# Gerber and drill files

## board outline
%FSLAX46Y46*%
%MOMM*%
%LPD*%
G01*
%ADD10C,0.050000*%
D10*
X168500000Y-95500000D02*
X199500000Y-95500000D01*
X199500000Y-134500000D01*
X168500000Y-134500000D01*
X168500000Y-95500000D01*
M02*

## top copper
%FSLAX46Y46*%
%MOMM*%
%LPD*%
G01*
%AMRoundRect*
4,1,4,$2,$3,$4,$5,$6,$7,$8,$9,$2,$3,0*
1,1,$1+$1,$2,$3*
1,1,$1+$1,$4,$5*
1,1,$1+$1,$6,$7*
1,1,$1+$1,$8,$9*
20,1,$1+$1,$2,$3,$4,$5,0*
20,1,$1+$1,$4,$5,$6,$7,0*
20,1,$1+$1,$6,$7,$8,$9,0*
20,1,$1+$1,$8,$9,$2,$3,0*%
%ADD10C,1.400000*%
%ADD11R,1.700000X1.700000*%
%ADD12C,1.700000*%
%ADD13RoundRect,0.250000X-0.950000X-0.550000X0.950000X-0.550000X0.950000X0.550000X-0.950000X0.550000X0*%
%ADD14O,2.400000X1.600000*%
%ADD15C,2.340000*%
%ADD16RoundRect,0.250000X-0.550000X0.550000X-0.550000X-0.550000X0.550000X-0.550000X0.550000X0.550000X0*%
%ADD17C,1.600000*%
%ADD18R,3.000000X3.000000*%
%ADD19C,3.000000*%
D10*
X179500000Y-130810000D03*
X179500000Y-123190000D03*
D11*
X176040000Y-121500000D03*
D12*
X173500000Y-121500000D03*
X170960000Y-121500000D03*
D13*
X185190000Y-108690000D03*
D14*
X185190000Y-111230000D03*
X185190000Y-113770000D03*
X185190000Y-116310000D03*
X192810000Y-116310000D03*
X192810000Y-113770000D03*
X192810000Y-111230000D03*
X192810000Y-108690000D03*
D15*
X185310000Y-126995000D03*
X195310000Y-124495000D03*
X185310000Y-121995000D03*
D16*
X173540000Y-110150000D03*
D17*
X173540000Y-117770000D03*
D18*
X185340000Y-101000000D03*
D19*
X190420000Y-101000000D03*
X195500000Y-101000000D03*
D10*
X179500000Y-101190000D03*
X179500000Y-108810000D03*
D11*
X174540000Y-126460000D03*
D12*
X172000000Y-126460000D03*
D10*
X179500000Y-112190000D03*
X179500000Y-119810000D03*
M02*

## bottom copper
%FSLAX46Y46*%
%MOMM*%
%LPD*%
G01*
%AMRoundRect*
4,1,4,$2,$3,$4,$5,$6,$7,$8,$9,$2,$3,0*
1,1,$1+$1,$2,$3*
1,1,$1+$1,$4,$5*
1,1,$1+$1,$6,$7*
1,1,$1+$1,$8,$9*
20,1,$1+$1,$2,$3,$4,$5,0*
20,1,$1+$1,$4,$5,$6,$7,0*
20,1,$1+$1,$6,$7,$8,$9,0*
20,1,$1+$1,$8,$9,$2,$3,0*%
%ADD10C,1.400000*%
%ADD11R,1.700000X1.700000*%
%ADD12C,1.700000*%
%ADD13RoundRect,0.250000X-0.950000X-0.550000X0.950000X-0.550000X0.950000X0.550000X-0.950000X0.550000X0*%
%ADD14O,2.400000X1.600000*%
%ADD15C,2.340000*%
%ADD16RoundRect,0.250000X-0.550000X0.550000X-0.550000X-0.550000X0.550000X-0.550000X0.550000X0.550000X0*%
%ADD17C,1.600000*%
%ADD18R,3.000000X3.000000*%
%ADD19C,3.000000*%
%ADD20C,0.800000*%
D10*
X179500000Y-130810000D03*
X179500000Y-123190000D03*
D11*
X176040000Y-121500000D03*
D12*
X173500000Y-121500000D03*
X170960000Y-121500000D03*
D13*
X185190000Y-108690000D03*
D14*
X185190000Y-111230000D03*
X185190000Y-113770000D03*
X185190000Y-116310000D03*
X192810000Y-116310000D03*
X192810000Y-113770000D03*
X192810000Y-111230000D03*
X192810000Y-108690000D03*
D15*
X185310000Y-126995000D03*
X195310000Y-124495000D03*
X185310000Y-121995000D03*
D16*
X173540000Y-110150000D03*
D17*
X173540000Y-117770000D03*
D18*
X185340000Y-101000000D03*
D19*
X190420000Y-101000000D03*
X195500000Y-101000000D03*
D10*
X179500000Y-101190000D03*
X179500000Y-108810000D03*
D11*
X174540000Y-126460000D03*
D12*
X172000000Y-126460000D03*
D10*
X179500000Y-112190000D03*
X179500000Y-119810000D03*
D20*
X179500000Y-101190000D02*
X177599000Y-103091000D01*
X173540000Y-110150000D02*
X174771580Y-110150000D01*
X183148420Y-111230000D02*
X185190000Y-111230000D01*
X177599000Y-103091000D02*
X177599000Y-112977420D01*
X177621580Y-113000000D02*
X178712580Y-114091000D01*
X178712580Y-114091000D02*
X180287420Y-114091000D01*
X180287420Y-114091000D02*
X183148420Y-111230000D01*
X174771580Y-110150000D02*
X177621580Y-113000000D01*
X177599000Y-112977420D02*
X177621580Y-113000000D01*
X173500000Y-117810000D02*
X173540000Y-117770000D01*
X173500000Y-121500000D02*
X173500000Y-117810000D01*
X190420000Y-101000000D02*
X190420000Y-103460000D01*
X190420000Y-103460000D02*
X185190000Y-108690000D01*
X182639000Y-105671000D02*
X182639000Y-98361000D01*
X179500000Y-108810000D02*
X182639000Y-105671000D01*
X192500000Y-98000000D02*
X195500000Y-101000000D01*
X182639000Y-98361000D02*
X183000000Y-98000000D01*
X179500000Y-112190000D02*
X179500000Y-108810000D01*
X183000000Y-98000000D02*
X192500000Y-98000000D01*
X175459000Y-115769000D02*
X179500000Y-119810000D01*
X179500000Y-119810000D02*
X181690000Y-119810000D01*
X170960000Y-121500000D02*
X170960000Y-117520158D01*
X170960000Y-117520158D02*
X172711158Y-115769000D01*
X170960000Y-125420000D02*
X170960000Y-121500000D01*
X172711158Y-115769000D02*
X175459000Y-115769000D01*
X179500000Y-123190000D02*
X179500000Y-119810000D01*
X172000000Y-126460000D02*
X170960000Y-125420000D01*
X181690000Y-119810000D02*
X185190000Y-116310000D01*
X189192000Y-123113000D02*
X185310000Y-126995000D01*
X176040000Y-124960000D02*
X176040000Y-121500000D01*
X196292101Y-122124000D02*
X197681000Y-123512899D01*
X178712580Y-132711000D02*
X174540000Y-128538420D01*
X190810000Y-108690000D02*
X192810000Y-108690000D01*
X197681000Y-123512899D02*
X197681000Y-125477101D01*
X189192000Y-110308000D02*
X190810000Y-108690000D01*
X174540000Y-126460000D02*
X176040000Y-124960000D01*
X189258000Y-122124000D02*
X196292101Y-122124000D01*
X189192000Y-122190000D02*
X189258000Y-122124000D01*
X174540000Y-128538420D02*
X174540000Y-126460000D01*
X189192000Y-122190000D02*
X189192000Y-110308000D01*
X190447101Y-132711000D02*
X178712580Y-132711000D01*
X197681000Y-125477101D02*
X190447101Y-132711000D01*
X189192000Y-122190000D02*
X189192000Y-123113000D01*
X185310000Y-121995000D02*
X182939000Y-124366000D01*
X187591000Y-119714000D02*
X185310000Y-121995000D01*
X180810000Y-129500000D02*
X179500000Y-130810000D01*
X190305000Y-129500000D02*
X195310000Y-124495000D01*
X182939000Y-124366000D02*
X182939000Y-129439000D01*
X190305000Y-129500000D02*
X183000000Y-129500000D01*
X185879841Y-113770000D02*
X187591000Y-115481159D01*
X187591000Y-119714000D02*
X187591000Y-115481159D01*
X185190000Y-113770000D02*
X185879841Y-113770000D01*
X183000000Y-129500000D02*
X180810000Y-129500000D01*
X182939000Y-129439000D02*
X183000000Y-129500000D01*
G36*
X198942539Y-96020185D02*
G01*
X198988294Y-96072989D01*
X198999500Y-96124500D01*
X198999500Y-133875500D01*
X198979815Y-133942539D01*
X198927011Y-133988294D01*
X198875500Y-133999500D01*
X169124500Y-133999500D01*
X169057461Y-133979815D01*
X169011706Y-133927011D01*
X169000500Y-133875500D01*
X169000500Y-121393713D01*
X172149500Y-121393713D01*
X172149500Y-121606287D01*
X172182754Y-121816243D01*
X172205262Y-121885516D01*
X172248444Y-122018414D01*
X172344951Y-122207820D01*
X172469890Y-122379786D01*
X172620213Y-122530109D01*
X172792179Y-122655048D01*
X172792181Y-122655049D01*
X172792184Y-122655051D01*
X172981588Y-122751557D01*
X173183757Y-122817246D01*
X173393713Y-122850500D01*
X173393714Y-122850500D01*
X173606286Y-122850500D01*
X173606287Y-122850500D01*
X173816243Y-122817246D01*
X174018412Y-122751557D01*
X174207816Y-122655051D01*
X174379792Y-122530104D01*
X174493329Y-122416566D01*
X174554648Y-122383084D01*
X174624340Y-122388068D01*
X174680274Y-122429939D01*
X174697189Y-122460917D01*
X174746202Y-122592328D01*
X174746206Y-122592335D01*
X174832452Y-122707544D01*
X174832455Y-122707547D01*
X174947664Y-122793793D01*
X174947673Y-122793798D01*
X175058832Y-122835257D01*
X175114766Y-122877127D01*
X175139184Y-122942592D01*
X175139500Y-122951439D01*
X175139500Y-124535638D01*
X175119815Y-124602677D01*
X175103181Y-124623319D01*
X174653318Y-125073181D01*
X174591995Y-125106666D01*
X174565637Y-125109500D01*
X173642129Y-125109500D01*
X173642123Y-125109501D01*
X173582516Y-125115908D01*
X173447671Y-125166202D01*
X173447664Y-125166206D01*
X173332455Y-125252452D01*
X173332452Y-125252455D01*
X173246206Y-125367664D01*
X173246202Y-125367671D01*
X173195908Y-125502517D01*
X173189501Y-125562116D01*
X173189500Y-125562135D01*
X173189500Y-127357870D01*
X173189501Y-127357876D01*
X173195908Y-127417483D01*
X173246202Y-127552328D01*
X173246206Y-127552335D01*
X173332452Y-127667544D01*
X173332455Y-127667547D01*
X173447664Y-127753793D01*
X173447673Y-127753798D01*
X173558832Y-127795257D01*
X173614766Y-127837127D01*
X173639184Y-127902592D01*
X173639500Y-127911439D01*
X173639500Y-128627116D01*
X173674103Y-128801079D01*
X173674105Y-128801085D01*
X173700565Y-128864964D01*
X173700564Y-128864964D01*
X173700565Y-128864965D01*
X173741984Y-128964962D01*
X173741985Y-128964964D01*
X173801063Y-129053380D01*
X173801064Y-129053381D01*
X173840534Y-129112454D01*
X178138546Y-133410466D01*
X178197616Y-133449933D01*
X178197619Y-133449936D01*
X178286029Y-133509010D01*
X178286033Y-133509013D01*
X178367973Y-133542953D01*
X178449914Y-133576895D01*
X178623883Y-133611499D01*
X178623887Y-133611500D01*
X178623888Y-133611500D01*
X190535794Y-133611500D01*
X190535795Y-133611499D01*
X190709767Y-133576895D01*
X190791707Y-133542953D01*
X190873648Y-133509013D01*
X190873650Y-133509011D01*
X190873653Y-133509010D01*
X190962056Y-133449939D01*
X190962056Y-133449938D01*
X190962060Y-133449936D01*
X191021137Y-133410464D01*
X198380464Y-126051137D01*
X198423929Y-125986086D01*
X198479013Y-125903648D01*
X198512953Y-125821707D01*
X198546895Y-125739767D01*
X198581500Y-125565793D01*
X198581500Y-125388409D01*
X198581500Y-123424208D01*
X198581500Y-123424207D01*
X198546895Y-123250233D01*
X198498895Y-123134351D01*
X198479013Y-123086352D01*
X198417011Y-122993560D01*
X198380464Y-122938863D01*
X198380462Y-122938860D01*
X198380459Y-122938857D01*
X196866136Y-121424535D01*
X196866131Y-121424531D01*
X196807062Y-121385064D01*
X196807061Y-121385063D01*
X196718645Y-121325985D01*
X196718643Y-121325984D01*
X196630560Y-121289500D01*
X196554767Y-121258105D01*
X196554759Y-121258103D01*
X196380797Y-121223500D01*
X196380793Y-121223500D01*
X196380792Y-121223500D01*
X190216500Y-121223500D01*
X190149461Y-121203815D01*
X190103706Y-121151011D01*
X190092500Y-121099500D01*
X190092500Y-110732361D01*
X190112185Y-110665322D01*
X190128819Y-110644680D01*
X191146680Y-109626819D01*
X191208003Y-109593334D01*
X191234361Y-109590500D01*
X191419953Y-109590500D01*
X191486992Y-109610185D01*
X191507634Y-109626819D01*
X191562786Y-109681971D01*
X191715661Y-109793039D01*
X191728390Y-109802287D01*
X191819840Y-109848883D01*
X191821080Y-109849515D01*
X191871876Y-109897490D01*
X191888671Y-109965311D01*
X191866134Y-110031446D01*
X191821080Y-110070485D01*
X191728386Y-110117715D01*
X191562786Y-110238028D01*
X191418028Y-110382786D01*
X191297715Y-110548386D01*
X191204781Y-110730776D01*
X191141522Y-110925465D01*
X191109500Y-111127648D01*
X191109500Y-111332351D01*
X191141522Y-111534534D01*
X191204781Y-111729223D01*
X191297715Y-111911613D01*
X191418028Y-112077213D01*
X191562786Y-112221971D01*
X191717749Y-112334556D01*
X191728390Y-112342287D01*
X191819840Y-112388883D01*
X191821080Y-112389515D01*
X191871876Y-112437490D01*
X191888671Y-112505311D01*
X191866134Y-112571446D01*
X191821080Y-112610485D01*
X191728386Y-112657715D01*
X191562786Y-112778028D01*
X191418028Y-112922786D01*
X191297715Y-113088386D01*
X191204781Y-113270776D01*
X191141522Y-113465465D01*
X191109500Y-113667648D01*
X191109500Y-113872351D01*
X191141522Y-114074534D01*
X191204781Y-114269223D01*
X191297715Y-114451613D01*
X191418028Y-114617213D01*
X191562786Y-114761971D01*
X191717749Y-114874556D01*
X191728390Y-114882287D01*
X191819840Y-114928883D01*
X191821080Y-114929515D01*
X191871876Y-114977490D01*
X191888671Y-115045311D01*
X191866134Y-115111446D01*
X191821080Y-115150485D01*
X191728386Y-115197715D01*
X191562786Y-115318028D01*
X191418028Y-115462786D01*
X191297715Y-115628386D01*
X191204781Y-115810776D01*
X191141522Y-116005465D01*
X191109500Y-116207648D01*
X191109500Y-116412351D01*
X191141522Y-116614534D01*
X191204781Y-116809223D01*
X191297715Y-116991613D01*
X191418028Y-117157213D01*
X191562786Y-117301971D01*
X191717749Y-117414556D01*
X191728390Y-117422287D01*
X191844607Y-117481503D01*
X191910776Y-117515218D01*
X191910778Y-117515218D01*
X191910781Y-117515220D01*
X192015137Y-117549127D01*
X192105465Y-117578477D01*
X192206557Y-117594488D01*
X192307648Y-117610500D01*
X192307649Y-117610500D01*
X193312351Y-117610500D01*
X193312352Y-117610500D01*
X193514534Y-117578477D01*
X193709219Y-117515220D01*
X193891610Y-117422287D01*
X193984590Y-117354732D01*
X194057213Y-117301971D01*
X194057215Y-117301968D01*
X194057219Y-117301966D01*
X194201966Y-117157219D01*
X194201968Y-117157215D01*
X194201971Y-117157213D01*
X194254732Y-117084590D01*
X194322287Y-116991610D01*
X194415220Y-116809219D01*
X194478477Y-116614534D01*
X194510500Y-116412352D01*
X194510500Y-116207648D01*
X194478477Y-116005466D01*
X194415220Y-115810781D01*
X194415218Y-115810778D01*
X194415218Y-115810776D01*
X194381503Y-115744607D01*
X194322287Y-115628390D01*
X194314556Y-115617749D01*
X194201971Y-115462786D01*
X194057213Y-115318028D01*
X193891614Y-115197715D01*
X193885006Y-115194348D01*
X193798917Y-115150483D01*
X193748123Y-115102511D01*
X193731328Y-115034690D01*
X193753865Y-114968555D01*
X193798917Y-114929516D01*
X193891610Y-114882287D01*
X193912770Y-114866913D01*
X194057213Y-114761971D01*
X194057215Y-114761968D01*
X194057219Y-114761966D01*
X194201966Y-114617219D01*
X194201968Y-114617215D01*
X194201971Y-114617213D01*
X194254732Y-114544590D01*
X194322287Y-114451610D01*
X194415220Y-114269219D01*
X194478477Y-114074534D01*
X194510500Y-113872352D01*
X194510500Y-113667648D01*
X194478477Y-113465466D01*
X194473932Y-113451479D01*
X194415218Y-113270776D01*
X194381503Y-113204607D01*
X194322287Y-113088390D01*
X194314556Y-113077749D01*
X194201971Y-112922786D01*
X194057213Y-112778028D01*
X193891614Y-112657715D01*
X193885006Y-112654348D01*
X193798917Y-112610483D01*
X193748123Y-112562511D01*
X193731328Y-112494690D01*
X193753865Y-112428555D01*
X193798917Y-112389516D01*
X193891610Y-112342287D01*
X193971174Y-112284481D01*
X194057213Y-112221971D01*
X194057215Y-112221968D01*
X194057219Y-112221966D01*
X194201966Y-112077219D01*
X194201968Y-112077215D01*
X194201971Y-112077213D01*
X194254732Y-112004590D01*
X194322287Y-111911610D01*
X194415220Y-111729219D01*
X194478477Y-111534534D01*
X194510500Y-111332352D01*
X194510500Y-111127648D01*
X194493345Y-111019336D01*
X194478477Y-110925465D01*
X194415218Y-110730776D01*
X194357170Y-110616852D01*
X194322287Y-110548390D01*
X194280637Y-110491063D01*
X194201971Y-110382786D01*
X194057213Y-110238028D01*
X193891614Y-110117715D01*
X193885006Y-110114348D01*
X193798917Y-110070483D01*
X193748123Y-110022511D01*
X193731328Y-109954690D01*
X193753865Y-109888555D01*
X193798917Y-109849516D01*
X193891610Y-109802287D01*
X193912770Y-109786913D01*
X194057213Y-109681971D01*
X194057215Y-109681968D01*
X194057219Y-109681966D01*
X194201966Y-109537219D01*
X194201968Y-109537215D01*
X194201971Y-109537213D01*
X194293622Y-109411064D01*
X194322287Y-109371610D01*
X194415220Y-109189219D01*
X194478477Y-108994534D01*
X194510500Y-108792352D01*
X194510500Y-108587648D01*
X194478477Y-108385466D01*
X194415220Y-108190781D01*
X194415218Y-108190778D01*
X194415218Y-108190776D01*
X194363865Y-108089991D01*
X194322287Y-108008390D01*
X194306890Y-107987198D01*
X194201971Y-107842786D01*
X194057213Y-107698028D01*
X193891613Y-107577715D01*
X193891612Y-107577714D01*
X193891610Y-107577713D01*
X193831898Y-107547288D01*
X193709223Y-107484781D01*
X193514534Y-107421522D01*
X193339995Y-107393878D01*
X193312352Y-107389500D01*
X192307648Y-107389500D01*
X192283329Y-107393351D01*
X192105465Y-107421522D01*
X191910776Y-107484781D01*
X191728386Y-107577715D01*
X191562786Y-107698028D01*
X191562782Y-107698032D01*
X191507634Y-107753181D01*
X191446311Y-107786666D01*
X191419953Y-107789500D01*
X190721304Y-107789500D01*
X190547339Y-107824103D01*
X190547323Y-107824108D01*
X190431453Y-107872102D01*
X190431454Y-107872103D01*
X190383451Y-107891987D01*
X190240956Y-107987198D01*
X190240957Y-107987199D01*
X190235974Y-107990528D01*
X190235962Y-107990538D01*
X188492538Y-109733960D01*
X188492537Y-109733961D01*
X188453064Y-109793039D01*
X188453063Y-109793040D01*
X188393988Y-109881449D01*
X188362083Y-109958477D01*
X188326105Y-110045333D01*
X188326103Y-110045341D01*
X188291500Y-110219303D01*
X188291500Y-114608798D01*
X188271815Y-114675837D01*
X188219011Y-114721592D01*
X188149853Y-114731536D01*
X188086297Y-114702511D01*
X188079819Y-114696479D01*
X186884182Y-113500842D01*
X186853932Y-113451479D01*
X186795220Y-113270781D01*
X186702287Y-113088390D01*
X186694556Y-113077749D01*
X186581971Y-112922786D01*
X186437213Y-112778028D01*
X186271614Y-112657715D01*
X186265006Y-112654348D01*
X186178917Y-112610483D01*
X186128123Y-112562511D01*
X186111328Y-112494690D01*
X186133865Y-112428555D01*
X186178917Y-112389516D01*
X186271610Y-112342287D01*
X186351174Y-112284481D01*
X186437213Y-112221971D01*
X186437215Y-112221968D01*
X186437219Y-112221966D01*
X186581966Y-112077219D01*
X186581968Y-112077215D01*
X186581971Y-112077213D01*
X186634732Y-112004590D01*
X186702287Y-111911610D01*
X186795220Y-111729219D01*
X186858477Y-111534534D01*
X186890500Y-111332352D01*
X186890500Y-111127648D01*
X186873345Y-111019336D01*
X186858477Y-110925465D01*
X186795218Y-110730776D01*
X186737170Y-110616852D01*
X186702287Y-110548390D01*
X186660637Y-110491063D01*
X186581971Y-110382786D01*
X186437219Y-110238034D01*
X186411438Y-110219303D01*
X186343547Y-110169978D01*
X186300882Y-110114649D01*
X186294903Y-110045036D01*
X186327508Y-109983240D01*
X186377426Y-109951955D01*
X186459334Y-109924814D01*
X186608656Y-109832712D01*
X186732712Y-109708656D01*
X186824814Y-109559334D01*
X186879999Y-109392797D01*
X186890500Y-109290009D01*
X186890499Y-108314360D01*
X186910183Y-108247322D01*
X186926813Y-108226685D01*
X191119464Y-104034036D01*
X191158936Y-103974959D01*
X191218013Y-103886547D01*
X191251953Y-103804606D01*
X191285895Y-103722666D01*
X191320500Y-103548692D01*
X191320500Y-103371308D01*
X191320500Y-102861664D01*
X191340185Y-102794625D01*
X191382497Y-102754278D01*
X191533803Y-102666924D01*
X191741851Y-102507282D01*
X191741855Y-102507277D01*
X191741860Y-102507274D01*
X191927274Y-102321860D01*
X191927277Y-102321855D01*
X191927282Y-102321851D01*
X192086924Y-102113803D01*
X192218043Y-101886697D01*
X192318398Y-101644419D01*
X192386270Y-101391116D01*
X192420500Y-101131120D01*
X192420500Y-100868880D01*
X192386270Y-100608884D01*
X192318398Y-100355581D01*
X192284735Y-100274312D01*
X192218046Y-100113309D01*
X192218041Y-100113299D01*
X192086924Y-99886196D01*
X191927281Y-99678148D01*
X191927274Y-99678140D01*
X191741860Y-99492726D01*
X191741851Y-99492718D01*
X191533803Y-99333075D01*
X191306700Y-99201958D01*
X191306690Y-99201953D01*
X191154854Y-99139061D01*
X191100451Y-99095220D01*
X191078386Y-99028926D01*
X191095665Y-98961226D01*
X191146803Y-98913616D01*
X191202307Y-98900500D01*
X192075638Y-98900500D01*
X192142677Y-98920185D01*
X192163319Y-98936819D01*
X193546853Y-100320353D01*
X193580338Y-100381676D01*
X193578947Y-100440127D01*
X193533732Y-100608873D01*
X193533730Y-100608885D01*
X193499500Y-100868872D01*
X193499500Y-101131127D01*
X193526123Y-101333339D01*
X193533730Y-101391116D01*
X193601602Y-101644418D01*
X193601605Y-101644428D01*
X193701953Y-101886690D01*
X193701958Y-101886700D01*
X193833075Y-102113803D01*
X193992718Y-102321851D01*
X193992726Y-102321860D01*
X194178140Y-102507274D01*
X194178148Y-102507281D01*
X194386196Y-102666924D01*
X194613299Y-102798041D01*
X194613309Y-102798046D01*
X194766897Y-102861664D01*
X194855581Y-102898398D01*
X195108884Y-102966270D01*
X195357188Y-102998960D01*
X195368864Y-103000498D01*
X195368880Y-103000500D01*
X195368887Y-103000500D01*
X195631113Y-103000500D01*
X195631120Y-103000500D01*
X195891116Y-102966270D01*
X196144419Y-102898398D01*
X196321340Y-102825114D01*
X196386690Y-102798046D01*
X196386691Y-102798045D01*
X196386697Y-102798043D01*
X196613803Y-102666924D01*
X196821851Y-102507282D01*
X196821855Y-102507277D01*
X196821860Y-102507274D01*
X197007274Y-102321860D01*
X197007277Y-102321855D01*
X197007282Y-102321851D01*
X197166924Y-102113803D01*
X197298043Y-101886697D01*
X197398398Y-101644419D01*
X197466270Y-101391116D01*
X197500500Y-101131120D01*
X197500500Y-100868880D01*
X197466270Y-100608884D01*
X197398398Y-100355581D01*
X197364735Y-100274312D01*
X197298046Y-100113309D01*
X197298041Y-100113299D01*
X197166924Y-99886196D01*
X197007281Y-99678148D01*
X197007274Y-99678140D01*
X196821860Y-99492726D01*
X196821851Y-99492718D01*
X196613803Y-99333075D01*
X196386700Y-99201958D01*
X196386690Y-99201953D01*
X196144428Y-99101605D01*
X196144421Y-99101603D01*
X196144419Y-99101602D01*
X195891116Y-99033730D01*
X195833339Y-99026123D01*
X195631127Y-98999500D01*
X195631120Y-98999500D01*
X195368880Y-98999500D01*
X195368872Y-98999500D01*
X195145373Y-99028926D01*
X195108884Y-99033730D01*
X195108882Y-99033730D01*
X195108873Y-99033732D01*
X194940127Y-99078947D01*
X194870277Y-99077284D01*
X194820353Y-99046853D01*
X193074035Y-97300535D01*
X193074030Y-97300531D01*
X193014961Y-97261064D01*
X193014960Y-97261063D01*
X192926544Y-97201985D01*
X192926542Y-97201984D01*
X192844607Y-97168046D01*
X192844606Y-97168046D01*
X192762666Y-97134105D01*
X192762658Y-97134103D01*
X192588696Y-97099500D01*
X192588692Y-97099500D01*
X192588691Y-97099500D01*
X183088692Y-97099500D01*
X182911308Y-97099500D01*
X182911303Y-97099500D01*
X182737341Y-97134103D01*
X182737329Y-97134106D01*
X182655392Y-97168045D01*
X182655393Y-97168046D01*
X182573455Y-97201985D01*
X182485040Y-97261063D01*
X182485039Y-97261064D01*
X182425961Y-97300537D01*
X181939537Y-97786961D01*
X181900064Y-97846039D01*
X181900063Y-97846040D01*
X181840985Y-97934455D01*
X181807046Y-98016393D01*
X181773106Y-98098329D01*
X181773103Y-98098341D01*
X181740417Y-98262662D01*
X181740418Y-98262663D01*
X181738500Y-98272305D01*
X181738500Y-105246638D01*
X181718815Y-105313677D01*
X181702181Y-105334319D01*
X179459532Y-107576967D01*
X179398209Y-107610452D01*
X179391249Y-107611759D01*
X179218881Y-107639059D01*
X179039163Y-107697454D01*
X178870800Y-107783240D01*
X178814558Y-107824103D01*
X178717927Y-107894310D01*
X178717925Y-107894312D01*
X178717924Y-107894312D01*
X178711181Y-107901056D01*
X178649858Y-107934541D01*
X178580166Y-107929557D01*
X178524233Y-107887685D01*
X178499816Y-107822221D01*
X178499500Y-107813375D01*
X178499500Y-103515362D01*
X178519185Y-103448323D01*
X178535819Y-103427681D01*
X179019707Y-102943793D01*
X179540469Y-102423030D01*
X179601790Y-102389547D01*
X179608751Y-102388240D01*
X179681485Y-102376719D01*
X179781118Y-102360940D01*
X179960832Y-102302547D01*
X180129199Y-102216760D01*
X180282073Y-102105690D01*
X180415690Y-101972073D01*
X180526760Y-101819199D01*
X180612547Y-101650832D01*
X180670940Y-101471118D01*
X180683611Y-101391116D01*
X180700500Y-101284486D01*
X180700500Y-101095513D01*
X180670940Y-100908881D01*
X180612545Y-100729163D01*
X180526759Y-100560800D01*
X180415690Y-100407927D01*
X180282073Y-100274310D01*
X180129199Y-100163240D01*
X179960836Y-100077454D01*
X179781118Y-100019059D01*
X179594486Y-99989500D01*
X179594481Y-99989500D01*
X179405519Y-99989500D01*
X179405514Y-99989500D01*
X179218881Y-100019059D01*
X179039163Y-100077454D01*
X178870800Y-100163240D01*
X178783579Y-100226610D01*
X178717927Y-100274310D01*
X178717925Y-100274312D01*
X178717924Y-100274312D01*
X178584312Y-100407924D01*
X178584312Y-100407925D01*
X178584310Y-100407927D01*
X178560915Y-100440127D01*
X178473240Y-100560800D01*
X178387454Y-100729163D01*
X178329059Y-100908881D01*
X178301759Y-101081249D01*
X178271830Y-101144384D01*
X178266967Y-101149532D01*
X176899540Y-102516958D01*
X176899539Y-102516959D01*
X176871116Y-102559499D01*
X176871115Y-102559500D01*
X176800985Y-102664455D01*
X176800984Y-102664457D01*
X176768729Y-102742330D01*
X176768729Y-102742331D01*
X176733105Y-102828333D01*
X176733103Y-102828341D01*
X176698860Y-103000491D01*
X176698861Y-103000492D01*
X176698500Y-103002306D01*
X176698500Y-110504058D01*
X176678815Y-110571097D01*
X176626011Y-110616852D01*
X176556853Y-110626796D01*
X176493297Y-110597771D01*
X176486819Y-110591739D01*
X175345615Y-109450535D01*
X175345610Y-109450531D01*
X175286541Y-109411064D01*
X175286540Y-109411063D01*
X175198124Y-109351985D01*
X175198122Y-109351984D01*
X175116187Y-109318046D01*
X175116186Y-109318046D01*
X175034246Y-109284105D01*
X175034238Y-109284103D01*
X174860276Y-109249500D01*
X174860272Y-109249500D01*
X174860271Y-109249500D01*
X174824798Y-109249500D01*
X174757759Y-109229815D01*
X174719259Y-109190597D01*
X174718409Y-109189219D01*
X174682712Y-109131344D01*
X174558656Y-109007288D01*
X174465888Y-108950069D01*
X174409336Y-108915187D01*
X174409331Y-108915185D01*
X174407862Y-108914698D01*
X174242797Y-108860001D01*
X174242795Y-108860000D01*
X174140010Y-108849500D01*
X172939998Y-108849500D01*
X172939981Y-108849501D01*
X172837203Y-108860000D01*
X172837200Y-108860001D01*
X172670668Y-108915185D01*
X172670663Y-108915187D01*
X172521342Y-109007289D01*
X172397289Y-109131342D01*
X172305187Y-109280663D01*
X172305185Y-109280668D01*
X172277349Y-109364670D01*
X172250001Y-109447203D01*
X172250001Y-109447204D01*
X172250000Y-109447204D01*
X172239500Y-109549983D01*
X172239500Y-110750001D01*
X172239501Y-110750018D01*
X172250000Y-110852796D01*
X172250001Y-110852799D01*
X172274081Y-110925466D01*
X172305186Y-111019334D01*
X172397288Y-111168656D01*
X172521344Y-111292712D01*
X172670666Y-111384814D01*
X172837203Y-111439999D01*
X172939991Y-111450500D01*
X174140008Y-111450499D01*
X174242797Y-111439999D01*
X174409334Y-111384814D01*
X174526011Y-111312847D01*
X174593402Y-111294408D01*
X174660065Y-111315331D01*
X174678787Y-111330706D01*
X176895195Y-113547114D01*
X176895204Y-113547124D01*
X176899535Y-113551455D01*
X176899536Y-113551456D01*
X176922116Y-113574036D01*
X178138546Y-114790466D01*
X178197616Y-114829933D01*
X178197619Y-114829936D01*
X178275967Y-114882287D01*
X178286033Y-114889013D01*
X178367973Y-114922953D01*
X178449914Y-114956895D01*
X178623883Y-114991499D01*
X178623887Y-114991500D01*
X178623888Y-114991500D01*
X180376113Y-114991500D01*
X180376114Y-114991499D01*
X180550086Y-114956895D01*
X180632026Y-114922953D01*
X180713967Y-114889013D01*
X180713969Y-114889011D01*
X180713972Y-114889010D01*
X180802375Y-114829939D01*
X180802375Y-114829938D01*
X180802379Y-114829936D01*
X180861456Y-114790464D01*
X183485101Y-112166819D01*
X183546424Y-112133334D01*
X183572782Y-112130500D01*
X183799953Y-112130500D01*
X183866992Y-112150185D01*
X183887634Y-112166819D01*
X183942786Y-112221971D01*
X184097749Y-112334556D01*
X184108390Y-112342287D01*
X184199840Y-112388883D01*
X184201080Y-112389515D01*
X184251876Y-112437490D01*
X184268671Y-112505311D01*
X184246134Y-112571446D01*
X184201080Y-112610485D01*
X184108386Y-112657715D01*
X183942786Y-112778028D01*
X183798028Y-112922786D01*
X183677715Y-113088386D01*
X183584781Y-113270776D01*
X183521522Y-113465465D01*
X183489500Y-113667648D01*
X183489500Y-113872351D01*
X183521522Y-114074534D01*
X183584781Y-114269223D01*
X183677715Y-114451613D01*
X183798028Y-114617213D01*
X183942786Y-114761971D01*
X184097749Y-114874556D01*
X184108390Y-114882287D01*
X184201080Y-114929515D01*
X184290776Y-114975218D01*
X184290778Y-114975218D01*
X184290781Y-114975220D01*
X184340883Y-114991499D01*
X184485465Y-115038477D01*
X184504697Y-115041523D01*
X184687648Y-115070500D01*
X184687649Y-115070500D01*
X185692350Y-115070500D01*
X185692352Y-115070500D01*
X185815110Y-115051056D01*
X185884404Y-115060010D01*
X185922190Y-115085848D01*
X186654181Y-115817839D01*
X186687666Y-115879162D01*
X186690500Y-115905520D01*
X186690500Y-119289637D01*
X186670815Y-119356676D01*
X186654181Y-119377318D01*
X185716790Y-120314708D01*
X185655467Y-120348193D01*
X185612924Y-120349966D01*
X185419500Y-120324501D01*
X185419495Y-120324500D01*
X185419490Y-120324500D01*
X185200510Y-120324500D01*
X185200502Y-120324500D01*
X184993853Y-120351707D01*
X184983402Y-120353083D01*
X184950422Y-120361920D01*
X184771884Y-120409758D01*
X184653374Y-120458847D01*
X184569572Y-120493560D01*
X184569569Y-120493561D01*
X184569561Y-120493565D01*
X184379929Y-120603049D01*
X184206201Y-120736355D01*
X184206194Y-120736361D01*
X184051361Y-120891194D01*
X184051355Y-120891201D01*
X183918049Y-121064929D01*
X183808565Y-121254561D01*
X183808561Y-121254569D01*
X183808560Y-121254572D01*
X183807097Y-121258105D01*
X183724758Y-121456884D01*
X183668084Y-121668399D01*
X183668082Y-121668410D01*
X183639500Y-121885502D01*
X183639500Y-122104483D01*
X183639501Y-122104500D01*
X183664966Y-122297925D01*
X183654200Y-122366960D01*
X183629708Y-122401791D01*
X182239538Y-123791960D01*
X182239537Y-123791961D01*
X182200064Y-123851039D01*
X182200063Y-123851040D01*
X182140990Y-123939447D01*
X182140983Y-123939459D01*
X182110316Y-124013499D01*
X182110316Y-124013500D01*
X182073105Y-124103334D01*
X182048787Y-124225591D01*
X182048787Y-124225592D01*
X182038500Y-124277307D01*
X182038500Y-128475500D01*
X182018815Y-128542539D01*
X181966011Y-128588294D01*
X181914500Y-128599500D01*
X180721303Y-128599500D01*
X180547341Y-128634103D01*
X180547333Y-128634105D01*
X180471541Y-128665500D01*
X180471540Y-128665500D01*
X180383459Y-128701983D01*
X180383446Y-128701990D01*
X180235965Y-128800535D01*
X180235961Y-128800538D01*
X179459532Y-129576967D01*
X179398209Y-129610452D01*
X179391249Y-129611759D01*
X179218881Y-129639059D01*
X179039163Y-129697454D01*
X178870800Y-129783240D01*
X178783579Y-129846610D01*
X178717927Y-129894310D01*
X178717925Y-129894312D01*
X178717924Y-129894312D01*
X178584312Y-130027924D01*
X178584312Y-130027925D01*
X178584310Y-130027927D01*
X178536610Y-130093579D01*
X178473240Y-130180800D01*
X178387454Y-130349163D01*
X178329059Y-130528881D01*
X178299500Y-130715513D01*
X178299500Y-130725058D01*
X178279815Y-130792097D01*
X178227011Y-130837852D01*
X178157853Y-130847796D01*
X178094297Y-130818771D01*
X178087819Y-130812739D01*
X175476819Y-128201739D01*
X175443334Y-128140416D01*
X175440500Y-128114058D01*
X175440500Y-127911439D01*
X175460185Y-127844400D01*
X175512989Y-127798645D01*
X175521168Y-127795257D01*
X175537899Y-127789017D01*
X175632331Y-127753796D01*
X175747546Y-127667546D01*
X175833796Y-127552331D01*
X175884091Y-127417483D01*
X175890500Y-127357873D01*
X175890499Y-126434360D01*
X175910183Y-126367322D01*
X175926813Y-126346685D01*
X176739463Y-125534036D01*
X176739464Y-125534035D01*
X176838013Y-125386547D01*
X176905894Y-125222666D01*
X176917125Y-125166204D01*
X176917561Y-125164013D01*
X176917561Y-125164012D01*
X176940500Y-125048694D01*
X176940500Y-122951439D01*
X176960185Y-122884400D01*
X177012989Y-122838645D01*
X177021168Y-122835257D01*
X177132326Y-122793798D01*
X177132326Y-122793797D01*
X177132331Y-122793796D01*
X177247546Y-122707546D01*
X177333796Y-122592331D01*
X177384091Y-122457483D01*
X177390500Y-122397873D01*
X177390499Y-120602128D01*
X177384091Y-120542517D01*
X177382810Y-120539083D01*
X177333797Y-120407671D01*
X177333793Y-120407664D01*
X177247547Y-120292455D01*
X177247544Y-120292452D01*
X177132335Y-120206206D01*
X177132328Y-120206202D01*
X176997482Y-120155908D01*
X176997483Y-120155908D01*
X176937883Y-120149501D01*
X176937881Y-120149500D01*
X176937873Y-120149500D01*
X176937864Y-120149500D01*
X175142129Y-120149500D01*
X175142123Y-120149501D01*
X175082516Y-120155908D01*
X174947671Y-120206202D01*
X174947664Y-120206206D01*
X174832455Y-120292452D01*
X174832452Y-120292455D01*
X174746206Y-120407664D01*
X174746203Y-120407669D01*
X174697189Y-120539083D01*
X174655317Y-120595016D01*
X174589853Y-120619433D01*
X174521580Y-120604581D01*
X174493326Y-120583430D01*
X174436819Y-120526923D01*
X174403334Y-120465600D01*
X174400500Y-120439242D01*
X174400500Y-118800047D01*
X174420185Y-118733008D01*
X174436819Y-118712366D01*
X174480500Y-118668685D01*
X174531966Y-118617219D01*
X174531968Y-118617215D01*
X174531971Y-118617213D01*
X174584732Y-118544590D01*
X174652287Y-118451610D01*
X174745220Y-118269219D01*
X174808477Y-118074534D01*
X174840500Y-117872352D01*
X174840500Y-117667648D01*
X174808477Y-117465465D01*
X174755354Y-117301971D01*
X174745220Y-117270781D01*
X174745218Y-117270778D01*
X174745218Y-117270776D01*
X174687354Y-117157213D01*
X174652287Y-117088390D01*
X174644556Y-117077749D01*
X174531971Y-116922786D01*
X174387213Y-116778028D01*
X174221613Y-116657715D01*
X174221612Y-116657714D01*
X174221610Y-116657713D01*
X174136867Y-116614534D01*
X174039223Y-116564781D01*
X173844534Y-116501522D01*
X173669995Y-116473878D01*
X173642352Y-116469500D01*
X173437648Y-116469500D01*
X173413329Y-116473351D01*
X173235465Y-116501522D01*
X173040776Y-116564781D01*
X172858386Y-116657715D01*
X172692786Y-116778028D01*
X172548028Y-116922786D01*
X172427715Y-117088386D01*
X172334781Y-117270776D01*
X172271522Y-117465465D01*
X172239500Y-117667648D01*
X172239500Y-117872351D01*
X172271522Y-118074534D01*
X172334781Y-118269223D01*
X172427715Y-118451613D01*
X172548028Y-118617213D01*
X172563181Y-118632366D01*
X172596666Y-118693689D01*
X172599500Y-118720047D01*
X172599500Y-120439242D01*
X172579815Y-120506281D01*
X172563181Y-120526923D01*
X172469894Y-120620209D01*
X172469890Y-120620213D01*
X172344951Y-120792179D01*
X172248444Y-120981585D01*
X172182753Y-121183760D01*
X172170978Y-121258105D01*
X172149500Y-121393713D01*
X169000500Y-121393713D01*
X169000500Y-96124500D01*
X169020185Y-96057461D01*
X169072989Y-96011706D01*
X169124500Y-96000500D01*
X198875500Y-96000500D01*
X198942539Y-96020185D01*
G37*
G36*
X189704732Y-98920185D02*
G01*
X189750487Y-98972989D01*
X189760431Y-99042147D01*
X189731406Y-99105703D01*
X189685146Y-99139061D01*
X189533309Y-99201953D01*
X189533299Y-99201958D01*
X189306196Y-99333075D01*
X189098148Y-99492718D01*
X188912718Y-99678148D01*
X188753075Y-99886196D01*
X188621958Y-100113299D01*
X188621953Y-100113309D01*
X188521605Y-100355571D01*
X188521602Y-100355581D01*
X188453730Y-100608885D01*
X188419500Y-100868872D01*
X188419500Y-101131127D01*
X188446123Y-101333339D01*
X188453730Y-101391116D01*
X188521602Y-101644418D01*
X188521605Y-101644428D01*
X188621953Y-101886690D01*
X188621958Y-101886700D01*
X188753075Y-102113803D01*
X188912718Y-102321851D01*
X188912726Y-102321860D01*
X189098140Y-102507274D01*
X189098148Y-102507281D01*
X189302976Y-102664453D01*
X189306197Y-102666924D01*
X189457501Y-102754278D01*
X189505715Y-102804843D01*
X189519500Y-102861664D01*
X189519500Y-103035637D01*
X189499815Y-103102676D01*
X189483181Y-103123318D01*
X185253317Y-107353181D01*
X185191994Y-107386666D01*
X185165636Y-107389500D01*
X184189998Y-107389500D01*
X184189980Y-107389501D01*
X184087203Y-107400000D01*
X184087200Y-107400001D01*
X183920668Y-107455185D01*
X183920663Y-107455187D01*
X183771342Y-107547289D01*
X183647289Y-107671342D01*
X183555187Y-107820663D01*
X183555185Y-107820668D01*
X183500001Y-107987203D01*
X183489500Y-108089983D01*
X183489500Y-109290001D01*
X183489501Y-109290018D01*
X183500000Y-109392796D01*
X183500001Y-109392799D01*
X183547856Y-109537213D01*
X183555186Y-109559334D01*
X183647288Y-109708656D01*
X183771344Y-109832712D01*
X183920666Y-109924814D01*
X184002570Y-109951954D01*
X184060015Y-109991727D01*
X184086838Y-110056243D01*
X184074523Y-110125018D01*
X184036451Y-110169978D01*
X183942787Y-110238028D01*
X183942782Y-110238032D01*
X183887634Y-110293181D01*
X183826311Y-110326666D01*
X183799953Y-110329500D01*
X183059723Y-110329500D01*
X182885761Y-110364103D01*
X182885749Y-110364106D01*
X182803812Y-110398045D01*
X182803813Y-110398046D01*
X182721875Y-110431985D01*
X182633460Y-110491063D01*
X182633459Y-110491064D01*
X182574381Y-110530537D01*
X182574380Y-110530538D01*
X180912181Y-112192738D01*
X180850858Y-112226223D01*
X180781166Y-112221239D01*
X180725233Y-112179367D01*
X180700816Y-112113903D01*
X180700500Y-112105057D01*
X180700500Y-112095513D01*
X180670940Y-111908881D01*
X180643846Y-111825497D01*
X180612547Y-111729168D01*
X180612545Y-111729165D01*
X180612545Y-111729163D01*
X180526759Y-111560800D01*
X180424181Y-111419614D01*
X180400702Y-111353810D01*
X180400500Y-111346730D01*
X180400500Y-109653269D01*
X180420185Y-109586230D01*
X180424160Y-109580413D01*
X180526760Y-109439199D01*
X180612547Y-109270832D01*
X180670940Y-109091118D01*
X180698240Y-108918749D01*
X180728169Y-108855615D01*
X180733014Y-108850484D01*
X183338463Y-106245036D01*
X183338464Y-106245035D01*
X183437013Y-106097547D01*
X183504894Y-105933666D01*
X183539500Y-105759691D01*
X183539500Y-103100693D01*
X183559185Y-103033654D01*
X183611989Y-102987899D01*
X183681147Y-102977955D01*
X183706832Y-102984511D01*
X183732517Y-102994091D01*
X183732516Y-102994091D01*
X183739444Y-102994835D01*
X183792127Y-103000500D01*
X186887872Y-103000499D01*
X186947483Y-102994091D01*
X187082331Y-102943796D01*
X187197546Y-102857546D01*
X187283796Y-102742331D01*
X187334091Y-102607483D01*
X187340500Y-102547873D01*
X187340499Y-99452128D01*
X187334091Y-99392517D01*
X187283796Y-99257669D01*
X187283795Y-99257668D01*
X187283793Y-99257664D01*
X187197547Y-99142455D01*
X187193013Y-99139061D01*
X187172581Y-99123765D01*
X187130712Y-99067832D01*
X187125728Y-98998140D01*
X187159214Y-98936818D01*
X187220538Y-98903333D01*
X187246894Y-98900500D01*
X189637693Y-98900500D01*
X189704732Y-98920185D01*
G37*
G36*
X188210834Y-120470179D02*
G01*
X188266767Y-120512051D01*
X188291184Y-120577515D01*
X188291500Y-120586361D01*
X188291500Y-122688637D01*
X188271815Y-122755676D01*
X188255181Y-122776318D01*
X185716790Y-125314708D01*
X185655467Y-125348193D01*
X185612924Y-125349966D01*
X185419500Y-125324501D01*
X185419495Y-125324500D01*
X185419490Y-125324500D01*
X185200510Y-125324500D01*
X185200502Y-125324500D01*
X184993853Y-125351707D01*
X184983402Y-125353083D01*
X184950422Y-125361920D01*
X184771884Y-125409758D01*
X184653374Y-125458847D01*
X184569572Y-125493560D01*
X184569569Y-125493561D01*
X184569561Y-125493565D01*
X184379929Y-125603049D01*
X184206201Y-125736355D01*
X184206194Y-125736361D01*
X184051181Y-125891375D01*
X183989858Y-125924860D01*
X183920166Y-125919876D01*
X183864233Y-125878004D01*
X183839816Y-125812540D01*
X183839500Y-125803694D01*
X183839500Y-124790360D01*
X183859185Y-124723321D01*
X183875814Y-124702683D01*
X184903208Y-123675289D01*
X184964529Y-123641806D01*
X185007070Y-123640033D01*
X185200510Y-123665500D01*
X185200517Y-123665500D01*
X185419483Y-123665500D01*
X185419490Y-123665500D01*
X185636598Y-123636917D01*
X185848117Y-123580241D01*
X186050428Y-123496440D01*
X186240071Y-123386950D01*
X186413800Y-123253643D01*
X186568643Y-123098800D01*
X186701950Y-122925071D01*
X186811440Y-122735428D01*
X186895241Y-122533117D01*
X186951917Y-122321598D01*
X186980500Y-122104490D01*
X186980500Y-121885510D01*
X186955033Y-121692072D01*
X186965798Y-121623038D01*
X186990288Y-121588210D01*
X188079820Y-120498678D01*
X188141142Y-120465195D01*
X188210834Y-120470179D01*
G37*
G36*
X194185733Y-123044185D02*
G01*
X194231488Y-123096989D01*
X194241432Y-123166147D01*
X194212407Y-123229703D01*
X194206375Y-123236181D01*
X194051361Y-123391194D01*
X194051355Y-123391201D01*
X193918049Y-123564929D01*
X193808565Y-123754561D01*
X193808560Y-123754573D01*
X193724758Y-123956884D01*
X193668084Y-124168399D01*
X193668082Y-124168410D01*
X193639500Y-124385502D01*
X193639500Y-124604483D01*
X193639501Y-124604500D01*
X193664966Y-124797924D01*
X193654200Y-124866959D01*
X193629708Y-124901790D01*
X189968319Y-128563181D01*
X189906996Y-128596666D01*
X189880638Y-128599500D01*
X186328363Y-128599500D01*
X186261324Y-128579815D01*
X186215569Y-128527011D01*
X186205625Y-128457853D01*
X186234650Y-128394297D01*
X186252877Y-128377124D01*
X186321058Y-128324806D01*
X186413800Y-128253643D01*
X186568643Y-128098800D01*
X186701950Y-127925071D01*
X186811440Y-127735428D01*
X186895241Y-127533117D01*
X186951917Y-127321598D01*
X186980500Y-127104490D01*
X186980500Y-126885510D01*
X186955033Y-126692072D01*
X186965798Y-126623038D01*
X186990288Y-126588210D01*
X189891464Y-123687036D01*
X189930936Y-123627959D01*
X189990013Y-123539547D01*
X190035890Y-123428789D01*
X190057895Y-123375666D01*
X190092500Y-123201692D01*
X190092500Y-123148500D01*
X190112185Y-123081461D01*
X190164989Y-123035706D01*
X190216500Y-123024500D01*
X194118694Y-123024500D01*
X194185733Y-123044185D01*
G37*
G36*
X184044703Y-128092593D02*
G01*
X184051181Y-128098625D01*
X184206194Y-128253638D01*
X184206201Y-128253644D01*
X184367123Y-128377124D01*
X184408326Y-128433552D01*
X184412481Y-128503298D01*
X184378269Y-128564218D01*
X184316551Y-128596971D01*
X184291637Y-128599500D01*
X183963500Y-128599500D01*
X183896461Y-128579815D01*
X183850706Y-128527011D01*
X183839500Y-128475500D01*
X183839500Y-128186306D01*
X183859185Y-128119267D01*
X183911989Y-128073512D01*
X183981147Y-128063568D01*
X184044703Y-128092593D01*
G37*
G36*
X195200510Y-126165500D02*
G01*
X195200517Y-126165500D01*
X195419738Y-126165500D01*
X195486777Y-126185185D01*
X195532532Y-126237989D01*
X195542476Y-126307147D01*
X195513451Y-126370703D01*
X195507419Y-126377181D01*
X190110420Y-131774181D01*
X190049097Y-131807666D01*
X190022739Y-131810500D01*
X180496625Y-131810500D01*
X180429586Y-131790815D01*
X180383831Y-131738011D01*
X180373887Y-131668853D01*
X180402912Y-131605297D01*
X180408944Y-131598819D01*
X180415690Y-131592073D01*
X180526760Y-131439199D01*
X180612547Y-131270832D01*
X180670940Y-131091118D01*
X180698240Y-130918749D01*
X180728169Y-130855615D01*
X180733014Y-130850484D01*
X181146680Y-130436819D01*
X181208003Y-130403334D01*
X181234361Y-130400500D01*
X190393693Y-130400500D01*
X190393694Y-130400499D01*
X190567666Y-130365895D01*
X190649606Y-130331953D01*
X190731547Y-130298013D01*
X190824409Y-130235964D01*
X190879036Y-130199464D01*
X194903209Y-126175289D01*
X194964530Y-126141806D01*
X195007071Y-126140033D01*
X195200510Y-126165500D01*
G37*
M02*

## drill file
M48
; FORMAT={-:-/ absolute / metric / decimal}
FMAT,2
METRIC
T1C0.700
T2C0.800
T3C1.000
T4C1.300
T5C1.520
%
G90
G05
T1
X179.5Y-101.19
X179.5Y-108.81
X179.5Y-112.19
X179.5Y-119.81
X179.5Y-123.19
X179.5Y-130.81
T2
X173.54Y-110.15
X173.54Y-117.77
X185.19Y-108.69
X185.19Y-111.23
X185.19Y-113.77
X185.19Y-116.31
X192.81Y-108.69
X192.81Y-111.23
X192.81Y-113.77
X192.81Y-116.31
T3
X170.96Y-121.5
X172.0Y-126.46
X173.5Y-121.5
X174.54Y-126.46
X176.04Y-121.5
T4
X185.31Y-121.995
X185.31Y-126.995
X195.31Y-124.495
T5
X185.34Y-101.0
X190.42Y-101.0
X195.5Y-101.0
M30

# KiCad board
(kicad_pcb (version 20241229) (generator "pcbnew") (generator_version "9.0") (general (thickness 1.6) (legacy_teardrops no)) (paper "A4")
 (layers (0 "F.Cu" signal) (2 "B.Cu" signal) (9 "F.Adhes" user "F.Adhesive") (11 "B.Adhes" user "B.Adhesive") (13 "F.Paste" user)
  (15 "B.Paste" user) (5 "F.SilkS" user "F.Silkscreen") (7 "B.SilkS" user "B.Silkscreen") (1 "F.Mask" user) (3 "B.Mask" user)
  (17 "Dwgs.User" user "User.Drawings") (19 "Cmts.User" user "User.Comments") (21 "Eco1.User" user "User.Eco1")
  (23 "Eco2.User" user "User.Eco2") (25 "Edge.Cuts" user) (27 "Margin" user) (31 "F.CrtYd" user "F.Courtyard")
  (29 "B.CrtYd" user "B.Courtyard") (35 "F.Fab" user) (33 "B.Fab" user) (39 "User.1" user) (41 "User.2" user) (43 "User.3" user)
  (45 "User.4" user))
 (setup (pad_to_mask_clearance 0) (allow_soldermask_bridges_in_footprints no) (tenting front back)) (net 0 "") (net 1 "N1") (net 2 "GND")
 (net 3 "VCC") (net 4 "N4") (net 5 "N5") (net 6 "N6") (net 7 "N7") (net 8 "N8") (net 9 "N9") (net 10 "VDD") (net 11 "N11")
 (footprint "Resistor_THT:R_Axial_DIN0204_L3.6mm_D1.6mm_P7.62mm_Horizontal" (layer "F.Cu") (at 179.5 130.81 90)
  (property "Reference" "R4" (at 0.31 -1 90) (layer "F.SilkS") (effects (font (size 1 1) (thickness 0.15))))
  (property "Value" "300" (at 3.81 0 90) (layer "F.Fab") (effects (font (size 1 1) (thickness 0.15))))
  (pad "1" thru_hole circle (at 0 0 90) (size 1.4 1.4) (drill 0.7) (layers "*.Cu" "*.Mask") (remove_unused_layers no) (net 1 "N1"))
  (pad "2" thru_hole circle (at 7.62 0 90) (size 1.4 1.4) (drill 0.7) (layers "*.Cu" "*.Mask") (remove_unused_layers no) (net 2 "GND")))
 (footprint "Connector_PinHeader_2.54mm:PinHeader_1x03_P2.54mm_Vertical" (layer "F.Cu") (at 176.04 121.5 -90)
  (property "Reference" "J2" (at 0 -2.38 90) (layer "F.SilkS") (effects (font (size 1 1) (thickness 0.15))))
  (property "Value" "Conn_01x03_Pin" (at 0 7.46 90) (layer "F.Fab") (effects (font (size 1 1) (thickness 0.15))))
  (pad "1" thru_hole rect (at 0 0 270) (size 1.7 1.7) (drill 1) (layers "*.Cu" "*.Mask") (remove_unused_layers no) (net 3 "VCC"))
  (pad "2" thru_hole circle (at 0 2.54 270) (size 1.7 1.7) (drill 1) (layers "*.Cu" "*.Mask") (remove_unused_layers no) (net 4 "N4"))
  (pad "3" thru_hole circle (at 0 5.08 270) (size 1.7 1.7) (drill 1) (layers "*.Cu" "*.Mask") (remove_unused_layers no) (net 2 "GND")))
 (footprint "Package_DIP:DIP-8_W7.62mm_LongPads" (layer "F.Cu") (at 185.19 108.69)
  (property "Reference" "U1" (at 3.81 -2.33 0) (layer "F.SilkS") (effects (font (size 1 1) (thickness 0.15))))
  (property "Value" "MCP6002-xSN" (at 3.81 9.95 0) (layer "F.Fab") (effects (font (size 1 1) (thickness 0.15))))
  (pad "1" thru_hole roundrect (at 0 0) (size 2.4 1.6) (drill 0.8) (layers "*.Cu" "*.Mask") (remove_unused_layers no)
   (roundrect_rratio 0.15625) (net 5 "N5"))
  (pad "2" thru_hole oval (at 0 2.54) (size 2.4 1.6) (drill 0.8) (layers "*.Cu" "*.Mask") (remove_unused_layers no) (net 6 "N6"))
  (pad "3" thru_hole oval (at 0 5.08) (size 2.4 1.6) (drill 0.8) (layers "*.Cu" "*.Mask") (remove_unused_layers no) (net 1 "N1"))
  (pad "4" thru_hole oval (at 0 7.62) (size 2.4 1.6) (drill 0.8) (layers "*.Cu" "*.Mask") (remove_unused_layers no) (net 2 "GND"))
  (pad "5" thru_hole oval (at 7.62 7.62) (size 2.4 1.6) (drill 0.8) (layers "*.Cu" "*.Mask") (remove_unused_layers no) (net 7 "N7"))
  (pad "6" thru_hole oval (at 7.62 5.08) (size 2.4 1.6) (drill 0.8) (layers "*.Cu" "*.Mask") (remove_unused_layers no) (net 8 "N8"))
  (pad "7" thru_hole oval (at 7.62 2.54) (size 2.4 1.6) (drill 0.8) (layers "*.Cu" "*.Mask") (remove_unused_layers no) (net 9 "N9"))
  (pad "8" thru_hole oval (at 7.62 0) (size 2.4 1.6) (drill 0.8) (layers "*.Cu" "*.Mask") (remove_unused_layers no) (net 3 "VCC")))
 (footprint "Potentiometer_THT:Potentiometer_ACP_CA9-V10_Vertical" (layer "F.Cu") (at 185.31 126.995)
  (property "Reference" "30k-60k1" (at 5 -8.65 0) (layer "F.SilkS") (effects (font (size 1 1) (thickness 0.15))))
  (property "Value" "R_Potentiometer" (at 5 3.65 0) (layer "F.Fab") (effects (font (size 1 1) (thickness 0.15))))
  (pad "1" thru_hole circle (at 0 0) (size 2.34 2.34) (drill 1.3) (layers "*.Cu" "*.Mask") (remove_unused_layers no) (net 3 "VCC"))
  (pad "2" thru_hole circle (at 10 -2.5) (size 2.34 2.34) (drill 1.3) (layers "*.Cu" "*.Mask") (remove_unused_layers no) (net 1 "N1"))
  (pad "3" thru_hole circle (at 0 -5) (size 2.34 2.34) (drill 1.3) (layers "*.Cu" "*.Mask") (remove_unused_layers no) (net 1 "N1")))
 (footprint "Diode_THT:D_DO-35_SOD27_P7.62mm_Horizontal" (layer "F.Cu") (at 173.54 110.15 -90)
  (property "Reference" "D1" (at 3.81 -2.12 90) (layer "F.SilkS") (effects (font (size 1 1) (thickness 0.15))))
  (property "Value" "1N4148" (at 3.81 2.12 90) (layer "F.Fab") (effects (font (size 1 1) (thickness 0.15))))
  (pad "1" thru_hole roundrect (at 0 0 270) (size 1.6 1.6) (drill 0.8) (layers "*.Cu" "*.Mask") (remove_unused_layers no)
   (roundrect_rratio 0.15625) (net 6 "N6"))
  (pad "2" thru_hole circle (at 7.62 0 270) (size 1.6 1.6) (drill 0.8) (layers "*.Cu" "*.Mask") (remove_unused_layers no) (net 4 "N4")))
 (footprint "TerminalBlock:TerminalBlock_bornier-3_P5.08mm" (layer "F.Cu") (at 185.34 101)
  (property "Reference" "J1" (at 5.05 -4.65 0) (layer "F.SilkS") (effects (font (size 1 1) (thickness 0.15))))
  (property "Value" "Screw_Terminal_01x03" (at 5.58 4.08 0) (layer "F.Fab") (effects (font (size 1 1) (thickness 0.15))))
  (pad "1" thru_hole rect (at 0 0) (size 3 3) (drill 1.52) (layers "*.Cu" "*.Mask") (remove_unused_layers no) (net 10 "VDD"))
  (pad "2" thru_hole circle (at 5.08 0) (size 3 3) (drill 1.52) (layers "*.Cu" "*.Mask") (remove_unused_layers no) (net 5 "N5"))
  (pad "3" thru_hole circle (at 10.16 0) (size 3 3) (drill 1.52) (layers "*.Cu" "*.Mask") (remove_unused_layers no) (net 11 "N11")))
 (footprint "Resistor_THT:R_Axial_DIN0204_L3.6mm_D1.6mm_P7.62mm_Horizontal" (layer "F.Cu") (at 179.5 101.19 -90)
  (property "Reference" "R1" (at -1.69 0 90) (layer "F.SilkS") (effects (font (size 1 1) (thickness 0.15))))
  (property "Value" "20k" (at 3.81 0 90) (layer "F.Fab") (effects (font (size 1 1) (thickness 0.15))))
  (pad "1" thru_hole circle (at 0 0 270) (size 1.4 1.4) (drill 0.7) (layers "*.Cu" "*.Mask") (remove_unused_layers no) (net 6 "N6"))
  (pad "2" thru_hole circle (at 7.62 0 270) (size 1.4 1.4) (drill 0.7) (layers "*.Cu" "*.Mask") (remove_unused_layers no) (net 11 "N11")))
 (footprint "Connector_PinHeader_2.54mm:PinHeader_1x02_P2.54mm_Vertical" (layer "F.Cu") (at 174.54 126.46 -90)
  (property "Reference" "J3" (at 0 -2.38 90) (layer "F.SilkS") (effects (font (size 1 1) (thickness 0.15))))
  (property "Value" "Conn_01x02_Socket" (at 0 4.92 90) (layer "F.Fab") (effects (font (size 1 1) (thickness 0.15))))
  (pad "1" thru_hole rect (at 0 0 270) (size 1.7 1.7) (drill 1) (layers "*.Cu" "*.Mask") (remove_unused_layers no) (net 3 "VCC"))
  (pad "2" thru_hole circle (at 0 2.54 270) (size 1.7 1.7) (drill 1) (layers "*.Cu" "*.Mask") (remove_unused_layers no) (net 2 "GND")))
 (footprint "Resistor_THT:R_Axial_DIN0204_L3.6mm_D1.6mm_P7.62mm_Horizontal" (layer "F.Cu") (at 179.5 112.19 -90)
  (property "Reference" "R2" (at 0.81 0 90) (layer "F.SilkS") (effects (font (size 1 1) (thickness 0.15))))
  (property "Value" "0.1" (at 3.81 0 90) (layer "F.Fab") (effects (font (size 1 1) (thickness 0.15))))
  (pad "1" thru_hole circle (at 0 0 270) (size 1.4 1.4) (drill 0.7) (layers "*.Cu" "*.Mask") (remove_unused_layers no) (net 11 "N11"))
  (pad "2" thru_hole circle (at 7.62 0 270) (size 1.4 1.4) (drill 0.7) (layers "*.Cu" "*.Mask") (remove_unused_layers no) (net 2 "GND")))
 (gr_rect (start 168.5 95.5) (end 199.5 134.5) (stroke (width 0.05) (type default)) (fill no) (layer "Edge.Cuts"))
 (segment (start 179.5 101.19) (end 177.599 103.091) (width 0.8) (layer "B.Cu") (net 6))
 (segment (start 173.54 110.15) (end 174.77158 110.15) (width 0.8) (layer "B.Cu") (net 6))
 (segment (start 183.14842 111.23) (end 185.19 111.23) (width 0.8) (layer "B.Cu") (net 6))
 (segment (start 177.599 103.091) (end 177.599 112.97742) (width 0.8) (layer "B.Cu") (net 6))
 (segment (start 177.62158 113) (end 178.71258 114.091) (width 0.8) (layer "B.Cu") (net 6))
 (segment (start 178.71258 114.091) (end 180.28742 114.091) (width 0.8) (layer "B.Cu") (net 6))
 (segment (start 180.28742 114.091) (end 183.14842 111.23) (width 0.8) (layer "B.Cu") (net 6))
 (segment (start 174.77158 110.15) (end 177.62158 113) (width 0.8) (layer "B.Cu") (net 6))
 (segment (start 177.599 112.97742) (end 177.62158 113) (width 0.8) (layer "B.Cu") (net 6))
 (segment (start 173.5 117.81) (end 173.54 117.77) (width 0.8) (layer "B.Cu") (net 4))
 (segment (start 173.5 121.5) (end 173.5 117.81) (width 0.8) (layer "B.Cu") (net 4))
 (segment (start 190.42 101) (end 190.42 103.46) (width 0.8) (layer "B.Cu") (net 5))
 (segment (start 190.42 103.46) (end 185.19 108.69) (width 0.8) (layer "B.Cu") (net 5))
 (segment (start 182.639 105.671) (end 182.639 98.361) (width 0.8) (layer "B.Cu") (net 11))
 (segment (start 179.5 108.81) (end 182.639 105.671) (width 0.8) (layer "B.Cu") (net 11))
 (segment (start 192.5 98) (end 195.5 101) (width 0.8) (layer "B.Cu") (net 11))
 (segment (start 182.639 98.361) (end 183 98) (width 0.8) (layer "B.Cu") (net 11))
 (segment (start 179.5 112.19) (end 179.5 108.81) (width 0.8) (layer "B.Cu") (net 11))
 (segment (start 183 98) (end 192.5 98) (width 0.8) (layer "B.Cu") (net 11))
 (segment (start 175.459 115.769) (end 179.5 119.81) (width 0.8) (layer "B.Cu") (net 2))
 (segment (start 179.5 119.81) (end 181.69 119.81) (width 0.8) (layer "B.Cu") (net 2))
 (segment (start 170.96 121.5) (end 170.96 117.520158) (width 0.8) (layer "B.Cu") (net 2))
 (segment (start 170.96 117.520158) (end 172.711158 115.769) (width 0.8) (layer "B.Cu") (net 2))
 (segment (start 170.96 125.42) (end 170.96 121.5) (width 0.8) (layer "B.Cu") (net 2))
 (segment (start 172.711158 115.769) (end 175.459 115.769) (width 0.8) (layer "B.Cu") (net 2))
 (segment (start 179.5 123.19) (end 179.5 119.81) (width 0.8) (layer "B.Cu") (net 2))
 (segment (start 172 126.46) (end 170.96 125.42) (width 0.8) (layer "B.Cu") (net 2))
 (segment (start 181.69 119.81) (end 185.19 116.31) (width 0.8) (layer "B.Cu") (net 2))
 (segment (start 189.192 123.113) (end 185.31 126.995) (width 0.8) (layer "B.Cu") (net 3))
 (segment (start 176.04 124.96) (end 176.04 121.5) (width 0.8) (layer "B.Cu") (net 3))
 (segment (start 196.292101 122.124) (end 197.681 123.512899) (width 0.8) (layer "B.Cu") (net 3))
 (segment (start 178.71258 132.711) (end 174.54 128.53842) (width 0.8) (layer "B.Cu") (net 3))
 (segment (start 190.81 108.69) (end 192.81 108.69) (width 0.8) (layer "B.Cu") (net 3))
 (segment (start 197.681 123.512899) (end 197.681 125.477101) (width 0.8) (layer "B.Cu") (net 3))
 (segment (start 189.192 110.308) (end 190.81 108.69) (width 0.8) (layer "B.Cu") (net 3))
 (segment (start 174.54 126.46) (end 176.04 124.96) (width 0.8) (layer "B.Cu") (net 3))
 (segment (start 189.258 122.124) (end 196.292101 122.124) (width 0.8) (layer "B.Cu") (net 3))
 (segment (start 189.192 122.19) (end 189.258 122.124) (width 0.8) (layer "B.Cu") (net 3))
 (segment (start 174.54 128.53842) (end 174.54 126.46) (width 0.8) (layer "B.Cu") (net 3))
 (segment (start 189.192 122.19) (end 189.192 110.308) (width 0.8) (layer "B.Cu") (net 3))
 (segment (start 190.447101 132.711) (end 178.71258 132.711) (width 0.8) (layer "B.Cu") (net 3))
 (segment (start 197.681 125.477101) (end 190.447101 132.711) (width 0.8) (layer "B.Cu") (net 3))
 (segment (start 189.192 122.19) (end 189.192 123.113) (width 0.8) (layer "B.Cu") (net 3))
 (segment (start 185.31 121.995) (end 182.939 124.366) (width 0.8) (layer "B.Cu") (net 1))
 (segment (start 187.591 119.714) (end 185.31 121.995) (width 0.8) (layer "B.Cu") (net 1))
 (segment (start 180.81 129.5) (end 179.5 130.81) (width 0.8) (layer "B.Cu") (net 1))
 (segment (start 190.305 129.5) (end 195.31 124.495) (width 0.8) (layer "B.Cu") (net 1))
 (segment (start 182.939 124.366) (end 182.939 129.439) (width 0.8) (layer "B.Cu") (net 1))
 (segment (start 190.305 129.5) (end 183 129.5) (width 0.8) (layer "B.Cu") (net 1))
 (segment (start 185.879841 113.77) (end 187.591 115.481159) (width 0.8) (layer "B.Cu") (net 1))
 (segment (start 187.591 119.714) (end 187.591 115.481159) (width 0.8) (layer "B.Cu") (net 1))
 (segment (start 185.19 113.77) (end 185.879841 113.77) (width 0.8) (layer "B.Cu") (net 1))
 (segment (start 183 129.5) (end 180.81 129.5) (width 0.8) (layer "B.Cu") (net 1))
 (segment (start 182.939 129.439) (end 183 129.5) (width 0.8) (layer "B.Cu") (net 1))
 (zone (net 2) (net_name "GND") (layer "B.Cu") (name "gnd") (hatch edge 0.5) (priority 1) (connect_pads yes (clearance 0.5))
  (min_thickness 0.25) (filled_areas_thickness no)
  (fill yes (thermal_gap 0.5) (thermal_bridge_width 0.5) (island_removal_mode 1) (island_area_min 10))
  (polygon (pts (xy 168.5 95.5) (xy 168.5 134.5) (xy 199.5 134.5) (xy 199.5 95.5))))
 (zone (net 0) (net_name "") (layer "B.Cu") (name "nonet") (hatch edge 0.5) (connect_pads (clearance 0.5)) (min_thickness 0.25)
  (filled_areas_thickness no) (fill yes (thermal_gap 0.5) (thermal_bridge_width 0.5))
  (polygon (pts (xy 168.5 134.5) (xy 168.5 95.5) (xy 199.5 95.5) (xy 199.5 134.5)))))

